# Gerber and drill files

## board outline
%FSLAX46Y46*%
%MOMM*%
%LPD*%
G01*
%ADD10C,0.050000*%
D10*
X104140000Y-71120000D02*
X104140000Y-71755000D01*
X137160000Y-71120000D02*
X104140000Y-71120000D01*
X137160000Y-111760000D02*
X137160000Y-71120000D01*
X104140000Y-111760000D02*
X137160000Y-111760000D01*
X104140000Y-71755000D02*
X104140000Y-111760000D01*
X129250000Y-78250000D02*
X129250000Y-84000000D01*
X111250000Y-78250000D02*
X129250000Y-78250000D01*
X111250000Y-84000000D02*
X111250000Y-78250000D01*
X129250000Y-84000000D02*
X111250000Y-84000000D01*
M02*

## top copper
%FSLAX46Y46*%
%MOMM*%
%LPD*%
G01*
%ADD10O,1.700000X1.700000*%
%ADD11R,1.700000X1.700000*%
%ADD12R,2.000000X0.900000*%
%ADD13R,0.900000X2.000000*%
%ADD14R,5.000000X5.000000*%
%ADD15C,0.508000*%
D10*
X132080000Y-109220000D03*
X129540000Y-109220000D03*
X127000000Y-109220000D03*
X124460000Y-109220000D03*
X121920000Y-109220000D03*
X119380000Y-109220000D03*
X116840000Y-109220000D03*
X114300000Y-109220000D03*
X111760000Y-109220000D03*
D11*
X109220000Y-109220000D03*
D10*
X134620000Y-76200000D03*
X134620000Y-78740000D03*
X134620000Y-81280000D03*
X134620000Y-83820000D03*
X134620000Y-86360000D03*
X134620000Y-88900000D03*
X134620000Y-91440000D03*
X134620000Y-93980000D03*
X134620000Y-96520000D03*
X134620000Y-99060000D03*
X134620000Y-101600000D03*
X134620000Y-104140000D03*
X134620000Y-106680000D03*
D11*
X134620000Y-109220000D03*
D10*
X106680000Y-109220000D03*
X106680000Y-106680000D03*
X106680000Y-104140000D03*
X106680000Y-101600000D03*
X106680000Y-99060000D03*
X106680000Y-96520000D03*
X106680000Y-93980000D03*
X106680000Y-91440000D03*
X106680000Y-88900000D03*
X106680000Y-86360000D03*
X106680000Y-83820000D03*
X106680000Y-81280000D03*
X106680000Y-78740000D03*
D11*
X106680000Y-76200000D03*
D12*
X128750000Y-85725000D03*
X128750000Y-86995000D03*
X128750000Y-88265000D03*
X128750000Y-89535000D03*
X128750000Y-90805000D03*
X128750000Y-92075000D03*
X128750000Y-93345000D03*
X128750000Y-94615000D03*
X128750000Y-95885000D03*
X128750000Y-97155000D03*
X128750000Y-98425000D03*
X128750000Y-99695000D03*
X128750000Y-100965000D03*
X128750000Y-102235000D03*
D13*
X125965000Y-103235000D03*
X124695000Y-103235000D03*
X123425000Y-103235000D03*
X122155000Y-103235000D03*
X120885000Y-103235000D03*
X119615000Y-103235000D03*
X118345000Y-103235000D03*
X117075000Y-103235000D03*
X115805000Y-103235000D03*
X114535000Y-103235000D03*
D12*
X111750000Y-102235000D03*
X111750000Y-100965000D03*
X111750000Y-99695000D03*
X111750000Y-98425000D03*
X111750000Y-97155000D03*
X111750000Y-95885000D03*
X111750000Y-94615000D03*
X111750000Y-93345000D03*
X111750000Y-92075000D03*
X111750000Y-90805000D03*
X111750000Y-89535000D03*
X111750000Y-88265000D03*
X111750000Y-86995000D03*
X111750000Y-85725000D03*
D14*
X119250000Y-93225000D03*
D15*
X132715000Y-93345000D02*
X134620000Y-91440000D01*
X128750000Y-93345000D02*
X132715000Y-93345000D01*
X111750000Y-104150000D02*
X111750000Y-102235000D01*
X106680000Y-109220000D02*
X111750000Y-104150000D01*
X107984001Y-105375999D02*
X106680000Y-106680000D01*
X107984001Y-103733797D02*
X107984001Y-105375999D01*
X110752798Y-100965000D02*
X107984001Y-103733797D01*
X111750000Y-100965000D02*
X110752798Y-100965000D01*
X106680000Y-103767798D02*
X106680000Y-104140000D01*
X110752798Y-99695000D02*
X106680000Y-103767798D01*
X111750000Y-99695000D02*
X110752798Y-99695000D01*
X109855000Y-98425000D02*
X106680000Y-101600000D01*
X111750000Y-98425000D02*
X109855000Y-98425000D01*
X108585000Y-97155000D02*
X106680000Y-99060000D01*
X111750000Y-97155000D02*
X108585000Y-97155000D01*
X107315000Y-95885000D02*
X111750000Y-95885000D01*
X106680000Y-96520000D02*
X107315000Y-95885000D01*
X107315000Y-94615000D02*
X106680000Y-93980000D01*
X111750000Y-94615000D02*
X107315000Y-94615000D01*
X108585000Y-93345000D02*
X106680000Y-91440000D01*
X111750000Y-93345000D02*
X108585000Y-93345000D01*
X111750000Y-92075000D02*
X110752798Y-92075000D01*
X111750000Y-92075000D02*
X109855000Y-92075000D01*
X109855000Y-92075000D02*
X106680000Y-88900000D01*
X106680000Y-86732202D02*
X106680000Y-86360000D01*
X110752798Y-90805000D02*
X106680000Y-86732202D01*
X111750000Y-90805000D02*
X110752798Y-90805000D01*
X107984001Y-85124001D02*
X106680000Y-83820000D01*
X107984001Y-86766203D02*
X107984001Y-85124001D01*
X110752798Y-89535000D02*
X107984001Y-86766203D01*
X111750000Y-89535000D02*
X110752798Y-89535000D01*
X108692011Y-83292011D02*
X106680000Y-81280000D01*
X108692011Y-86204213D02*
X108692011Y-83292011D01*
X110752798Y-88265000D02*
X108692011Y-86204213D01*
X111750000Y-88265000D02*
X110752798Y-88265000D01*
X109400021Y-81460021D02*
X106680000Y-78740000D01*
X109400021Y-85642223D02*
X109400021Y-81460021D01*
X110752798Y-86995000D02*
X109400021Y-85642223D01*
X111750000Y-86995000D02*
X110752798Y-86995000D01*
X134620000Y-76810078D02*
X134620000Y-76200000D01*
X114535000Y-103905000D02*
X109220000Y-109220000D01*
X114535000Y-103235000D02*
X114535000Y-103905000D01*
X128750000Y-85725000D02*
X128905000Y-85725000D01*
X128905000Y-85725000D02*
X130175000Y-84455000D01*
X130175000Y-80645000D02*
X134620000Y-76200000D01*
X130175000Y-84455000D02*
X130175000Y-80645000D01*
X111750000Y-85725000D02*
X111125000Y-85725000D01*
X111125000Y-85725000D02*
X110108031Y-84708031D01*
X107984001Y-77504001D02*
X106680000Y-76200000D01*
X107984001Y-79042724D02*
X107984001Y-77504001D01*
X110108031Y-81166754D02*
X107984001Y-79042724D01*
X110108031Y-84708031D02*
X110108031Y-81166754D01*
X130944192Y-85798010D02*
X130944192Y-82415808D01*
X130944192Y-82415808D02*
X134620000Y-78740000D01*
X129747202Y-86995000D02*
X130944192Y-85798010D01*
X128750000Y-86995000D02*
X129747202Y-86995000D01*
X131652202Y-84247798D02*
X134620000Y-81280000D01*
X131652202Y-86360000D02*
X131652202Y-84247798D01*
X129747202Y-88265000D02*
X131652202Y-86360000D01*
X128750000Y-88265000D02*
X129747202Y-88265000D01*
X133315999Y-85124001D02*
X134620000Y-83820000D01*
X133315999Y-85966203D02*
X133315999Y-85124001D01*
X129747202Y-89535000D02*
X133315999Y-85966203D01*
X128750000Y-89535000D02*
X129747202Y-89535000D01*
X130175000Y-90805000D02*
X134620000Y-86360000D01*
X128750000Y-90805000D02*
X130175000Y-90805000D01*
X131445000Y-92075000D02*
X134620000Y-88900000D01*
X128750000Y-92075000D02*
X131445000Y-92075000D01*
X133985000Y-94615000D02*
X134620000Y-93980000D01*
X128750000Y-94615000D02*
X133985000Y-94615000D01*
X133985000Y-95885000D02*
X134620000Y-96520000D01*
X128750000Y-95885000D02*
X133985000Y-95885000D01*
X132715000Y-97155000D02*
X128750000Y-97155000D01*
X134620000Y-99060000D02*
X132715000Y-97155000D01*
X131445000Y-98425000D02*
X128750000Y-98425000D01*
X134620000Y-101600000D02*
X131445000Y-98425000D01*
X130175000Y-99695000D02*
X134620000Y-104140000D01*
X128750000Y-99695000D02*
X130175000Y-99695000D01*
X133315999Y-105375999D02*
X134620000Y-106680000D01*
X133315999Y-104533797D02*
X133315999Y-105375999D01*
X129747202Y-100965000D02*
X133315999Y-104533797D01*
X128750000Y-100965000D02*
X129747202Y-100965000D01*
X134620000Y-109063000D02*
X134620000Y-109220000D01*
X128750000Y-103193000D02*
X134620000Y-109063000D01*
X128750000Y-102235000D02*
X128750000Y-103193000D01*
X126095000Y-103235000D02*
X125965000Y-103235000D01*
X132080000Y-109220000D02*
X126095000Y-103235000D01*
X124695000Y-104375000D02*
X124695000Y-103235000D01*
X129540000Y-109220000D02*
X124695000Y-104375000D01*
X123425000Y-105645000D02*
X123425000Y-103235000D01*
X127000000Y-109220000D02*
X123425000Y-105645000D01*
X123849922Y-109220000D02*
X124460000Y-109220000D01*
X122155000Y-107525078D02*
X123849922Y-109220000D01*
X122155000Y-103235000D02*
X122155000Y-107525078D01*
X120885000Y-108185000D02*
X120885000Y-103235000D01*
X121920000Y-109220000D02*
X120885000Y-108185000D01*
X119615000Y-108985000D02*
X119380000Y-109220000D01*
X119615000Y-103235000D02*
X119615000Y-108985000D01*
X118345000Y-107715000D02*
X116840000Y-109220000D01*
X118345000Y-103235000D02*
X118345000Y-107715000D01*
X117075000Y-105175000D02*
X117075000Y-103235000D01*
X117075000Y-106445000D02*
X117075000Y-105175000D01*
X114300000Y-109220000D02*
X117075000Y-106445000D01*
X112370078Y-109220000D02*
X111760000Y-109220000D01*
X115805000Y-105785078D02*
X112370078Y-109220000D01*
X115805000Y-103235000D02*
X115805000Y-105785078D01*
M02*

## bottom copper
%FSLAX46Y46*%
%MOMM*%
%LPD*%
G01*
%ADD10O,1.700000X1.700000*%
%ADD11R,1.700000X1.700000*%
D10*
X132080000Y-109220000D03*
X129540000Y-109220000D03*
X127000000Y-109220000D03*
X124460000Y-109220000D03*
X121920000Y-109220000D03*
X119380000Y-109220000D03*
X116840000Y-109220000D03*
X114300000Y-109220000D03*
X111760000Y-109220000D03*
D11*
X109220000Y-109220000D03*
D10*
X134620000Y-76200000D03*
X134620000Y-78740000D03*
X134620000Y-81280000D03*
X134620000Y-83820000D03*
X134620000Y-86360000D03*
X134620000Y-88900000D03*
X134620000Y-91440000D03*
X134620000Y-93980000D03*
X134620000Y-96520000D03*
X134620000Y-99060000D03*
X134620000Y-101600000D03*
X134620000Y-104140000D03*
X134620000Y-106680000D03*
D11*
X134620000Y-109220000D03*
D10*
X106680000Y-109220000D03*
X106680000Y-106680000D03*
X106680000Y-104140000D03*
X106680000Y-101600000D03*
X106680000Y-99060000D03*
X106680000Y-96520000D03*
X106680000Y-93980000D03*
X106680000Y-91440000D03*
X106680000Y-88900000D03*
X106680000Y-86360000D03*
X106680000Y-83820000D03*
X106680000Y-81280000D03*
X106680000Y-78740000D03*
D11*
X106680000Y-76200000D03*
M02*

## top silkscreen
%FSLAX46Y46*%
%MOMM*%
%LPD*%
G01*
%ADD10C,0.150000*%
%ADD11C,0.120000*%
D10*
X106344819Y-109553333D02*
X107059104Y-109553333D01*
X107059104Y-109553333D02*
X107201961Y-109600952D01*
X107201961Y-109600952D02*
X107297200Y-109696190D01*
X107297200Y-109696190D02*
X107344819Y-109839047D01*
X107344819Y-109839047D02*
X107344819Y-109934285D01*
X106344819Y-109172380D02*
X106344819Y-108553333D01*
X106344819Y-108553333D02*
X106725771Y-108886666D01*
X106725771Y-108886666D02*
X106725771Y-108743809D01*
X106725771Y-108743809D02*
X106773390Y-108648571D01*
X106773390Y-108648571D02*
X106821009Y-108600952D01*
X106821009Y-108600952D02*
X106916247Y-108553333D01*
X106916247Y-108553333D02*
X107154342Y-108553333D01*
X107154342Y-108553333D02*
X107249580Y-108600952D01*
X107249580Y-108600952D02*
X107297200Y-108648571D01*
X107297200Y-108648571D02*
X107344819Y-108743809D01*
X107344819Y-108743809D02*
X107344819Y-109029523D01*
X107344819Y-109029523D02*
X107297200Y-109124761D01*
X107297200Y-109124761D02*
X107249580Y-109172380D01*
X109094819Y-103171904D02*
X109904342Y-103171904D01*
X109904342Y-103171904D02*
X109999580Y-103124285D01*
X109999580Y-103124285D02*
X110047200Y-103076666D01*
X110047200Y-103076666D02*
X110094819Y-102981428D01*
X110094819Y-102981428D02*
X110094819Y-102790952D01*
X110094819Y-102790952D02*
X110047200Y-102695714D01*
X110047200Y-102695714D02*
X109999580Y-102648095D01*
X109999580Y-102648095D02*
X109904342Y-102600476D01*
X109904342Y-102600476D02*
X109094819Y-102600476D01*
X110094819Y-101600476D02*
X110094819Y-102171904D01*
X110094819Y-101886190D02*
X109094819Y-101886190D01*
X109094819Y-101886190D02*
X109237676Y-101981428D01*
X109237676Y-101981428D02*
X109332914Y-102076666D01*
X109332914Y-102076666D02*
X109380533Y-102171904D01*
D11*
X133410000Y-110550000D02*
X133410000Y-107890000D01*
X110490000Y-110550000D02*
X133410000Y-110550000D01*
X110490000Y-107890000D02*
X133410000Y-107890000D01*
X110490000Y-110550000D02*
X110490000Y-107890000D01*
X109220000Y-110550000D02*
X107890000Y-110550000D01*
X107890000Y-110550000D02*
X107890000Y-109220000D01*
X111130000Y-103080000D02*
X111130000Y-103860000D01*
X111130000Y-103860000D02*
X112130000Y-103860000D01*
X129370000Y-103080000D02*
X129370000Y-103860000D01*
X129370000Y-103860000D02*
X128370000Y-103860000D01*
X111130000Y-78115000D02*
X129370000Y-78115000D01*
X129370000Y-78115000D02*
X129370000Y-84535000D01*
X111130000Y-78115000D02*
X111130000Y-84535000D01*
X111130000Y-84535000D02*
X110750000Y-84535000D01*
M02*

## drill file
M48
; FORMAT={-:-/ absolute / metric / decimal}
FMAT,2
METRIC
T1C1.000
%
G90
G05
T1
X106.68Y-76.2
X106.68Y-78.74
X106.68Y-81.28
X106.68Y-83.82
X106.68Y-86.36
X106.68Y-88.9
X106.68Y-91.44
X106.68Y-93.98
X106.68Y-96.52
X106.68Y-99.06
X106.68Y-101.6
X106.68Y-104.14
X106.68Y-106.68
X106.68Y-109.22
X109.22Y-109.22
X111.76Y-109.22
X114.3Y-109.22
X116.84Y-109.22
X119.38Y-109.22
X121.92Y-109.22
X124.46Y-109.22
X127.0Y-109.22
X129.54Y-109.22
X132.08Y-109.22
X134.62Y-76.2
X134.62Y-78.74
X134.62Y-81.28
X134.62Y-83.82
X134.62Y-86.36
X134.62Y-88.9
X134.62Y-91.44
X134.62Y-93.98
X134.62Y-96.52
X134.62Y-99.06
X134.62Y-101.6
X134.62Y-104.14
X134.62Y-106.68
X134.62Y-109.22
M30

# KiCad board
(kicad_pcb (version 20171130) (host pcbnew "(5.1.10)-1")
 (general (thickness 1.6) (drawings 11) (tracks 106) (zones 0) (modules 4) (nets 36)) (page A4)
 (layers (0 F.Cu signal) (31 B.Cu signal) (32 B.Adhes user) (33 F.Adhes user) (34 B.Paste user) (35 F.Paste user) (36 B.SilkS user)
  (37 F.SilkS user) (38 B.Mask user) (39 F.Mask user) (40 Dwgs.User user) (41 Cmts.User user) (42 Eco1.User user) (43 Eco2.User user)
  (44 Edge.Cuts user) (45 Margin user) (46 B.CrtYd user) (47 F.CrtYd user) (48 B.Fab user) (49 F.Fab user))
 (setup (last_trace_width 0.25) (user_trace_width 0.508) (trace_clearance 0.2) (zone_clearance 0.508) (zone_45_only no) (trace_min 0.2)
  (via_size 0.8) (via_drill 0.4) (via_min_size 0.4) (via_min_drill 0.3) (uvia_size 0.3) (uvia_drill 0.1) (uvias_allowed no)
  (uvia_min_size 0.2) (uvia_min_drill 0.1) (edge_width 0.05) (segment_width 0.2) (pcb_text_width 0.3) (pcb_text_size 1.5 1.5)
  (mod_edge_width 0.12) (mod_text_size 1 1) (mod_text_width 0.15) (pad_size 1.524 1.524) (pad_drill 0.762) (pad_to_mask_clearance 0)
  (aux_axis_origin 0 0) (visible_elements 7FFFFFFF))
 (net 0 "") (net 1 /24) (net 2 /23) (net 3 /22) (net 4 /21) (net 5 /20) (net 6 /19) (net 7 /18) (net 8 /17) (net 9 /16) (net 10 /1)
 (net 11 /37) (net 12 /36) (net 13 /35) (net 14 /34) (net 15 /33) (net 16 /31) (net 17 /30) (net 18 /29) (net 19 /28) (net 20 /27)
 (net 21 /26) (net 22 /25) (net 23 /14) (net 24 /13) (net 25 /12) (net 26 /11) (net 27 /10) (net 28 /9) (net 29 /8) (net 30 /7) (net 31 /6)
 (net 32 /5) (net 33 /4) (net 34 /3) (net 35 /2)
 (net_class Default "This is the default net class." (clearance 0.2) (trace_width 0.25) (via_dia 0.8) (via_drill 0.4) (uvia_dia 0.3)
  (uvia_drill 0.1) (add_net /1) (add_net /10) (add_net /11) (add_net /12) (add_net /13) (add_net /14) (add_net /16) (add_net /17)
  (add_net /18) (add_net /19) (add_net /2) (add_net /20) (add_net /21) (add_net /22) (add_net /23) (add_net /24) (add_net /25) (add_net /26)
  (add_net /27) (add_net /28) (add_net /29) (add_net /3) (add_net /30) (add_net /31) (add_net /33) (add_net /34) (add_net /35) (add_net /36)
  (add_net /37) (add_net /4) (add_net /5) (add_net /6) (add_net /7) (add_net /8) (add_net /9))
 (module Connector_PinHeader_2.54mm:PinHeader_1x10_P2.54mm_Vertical (layer F.Cu) (at 109.22 109.22 90)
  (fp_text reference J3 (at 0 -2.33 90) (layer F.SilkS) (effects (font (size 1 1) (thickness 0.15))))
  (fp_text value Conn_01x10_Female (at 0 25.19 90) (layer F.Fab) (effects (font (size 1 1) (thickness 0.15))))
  (fp_line (start -1.33 24.19) (end 1.33 24.19) (layer F.SilkS) (width 0.12))
  (fp_line (start -1.33 1.27) (end -1.33 24.19) (layer F.SilkS) (width 0.12))
  (fp_line (start 1.33 1.27) (end 1.33 24.19) (layer F.SilkS) (width 0.12))
  (fp_line (start -1.33 1.27) (end 1.33 1.27) (layer F.SilkS) (width 0.12))
  (fp_line (start -1.33 0) (end -1.33 -1.33) (layer F.SilkS) (width 0.12))
  (fp_line (start -1.33 -1.33) (end 0 -1.33) (layer F.SilkS) (width 0.12))
  (pad 10 thru_hole oval (at 0 22.86 90) (size 1.7 1.7) (drill 1) (layers *.Cu *.Mask) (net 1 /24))
  (pad 9 thru_hole oval (at 0 20.32 90) (size 1.7 1.7) (drill 1) (layers *.Cu *.Mask) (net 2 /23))
  (pad 8 thru_hole oval (at 0 17.78 90) (size 1.7 1.7) (drill 1) (layers *.Cu *.Mask) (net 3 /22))
  (pad 7 thru_hole oval (at 0 15.24 90) (size 1.7 1.7) (drill 1) (layers *.Cu *.Mask) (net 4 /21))
  (pad 6 thru_hole oval (at 0 12.7 90) (size 1.7 1.7) (drill 1) (layers *.Cu *.Mask) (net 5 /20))
  (pad 5 thru_hole oval (at 0 10.16 90) (size 1.7 1.7) (drill 1) (layers *.Cu *.Mask) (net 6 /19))
  (pad 4 thru_hole oval (at 0 7.62 90) (size 1.7 1.7) (drill 1) (layers *.Cu *.Mask) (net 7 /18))
  (pad 3 thru_hole oval (at 0 5.08 90) (size 1.7 1.7) (drill 1) (layers *.Cu *.Mask) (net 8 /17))
  (pad 2 thru_hole oval (at 0 2.54 90) (size 1.7 1.7) (drill 1) (layers *.Cu *.Mask) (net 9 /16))
  (pad 1 thru_hole rect (at 0 0 90) (size 1.7 1.7) (drill 1) (layers *.Cu *.Mask) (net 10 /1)))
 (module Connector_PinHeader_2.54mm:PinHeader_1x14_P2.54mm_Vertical (layer B.Cu) (at 134.62 109.22)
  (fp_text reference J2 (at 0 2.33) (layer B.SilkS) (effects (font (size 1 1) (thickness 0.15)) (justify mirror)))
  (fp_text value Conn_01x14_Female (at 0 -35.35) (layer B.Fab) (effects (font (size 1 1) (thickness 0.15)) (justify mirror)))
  (pad 14 thru_hole oval (at 0 -33.02) (size 1.7 1.7) (drill 1) (layers *.Cu *.Mask) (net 10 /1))
  (pad 13 thru_hole oval (at 0 -30.48) (size 1.7 1.7) (drill 1) (layers *.Cu *.Mask) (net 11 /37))
  (pad 12 thru_hole oval (at 0 -27.94) (size 1.7 1.7) (drill 1) (layers *.Cu *.Mask) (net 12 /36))
  (pad 11 thru_hole oval (at 0 -25.4) (size 1.7 1.7) (drill 1) (layers *.Cu *.Mask) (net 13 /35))
  (pad 10 thru_hole oval (at 0 -22.86) (size 1.7 1.7) (drill 1) (layers *.Cu *.Mask) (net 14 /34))
  (pad 9 thru_hole oval (at 0 -20.32) (size 1.7 1.7) (drill 1) (layers *.Cu *.Mask) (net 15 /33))
  (pad 8 thru_hole oval (at 0 -17.78) (size 1.7 1.7) (drill 1) (layers *.Cu *.Mask))
  (pad 7 thru_hole oval (at 0 -15.24) (size 1.7 1.7) (drill 1) (layers *.Cu *.Mask) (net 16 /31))
  (pad 6 thru_hole oval (at 0 -12.7) (size 1.7 1.7) (drill 1) (layers *.Cu *.Mask) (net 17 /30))
  (pad 5 thru_hole oval (at 0 -10.16) (size 1.7 1.7) (drill 1) (layers *.Cu *.Mask) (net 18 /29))
  (pad 4 thru_hole oval (at 0 -7.62) (size 1.7 1.7) (drill 1) (layers *.Cu *.Mask) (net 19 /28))
  (pad 3 thru_hole oval (at 0 -5.08) (size 1.7 1.7) (drill 1) (layers *.Cu *.Mask) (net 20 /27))
  (pad 2 thru_hole oval (at 0 -2.54) (size 1.7 1.7) (drill 1) (layers *.Cu *.Mask) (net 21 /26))
  (pad 1 thru_hole rect (at 0 0) (size 1.7 1.7) (drill 1) (layers *.Cu *.Mask) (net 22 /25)))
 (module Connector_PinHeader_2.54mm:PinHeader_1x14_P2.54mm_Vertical (layer B.Cu) (at 106.68 76.2 180)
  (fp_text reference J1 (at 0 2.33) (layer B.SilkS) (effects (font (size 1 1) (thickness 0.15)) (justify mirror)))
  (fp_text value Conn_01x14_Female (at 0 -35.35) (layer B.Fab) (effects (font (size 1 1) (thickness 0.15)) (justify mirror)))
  (pad 14 thru_hole oval (at 0 -33.02 180) (size 1.7 1.7) (drill 1) (layers *.Cu *.Mask) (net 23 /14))
  (pad 13 thru_hole oval (at 0 -30.48 180) (size 1.7 1.7) (drill 1) (layers *.Cu *.Mask) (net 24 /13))
  (pad 12 thru_hole oval (at 0 -27.94 180) (size 1.7 1.7) (drill 1) (layers *.Cu *.Mask) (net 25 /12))
  (pad 11 thru_hole oval (at 0 -25.4 180) (size 1.7 1.7) (drill 1) (layers *.Cu *.Mask) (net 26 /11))
  (pad 10 thru_hole oval (at 0 -22.86 180) (size 1.7 1.7) (drill 1) (layers *.Cu *.Mask) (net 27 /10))
  (pad 9 thru_hole oval (at 0 -20.32 180) (size 1.7 1.7) (drill 1) (layers *.Cu *.Mask) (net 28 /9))
  (pad 8 thru_hole oval (at 0 -17.78 180) (size 1.7 1.7) (drill 1) (layers *.Cu *.Mask) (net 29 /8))
  (pad 7 thru_hole oval (at 0 -15.24 180) (size 1.7 1.7) (drill 1) (layers *.Cu *.Mask) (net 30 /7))
  (pad 6 thru_hole oval (at 0 -12.7 180) (size 1.7 1.7) (drill 1) (layers *.Cu *.Mask) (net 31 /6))
  (pad 5 thru_hole oval (at 0 -10.16 180) (size 1.7 1.7) (drill 1) (layers *.Cu *.Mask) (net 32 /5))
  (pad 4 thru_hole oval (at 0 -7.62 180) (size 1.7 1.7) (drill 1) (layers *.Cu *.Mask) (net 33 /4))
  (pad 3 thru_hole oval (at 0 -5.08 180) (size 1.7 1.7) (drill 1) (layers *.Cu *.Mask) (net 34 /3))
  (pad 2 thru_hole oval (at 0 -2.54 180) (size 1.7 1.7) (drill 1) (layers *.Cu *.Mask) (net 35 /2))
  (pad 1 thru_hole rect (at 0 0 180) (size 1.7 1.7) (drill 1) (layers *.Cu *.Mask) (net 10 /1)))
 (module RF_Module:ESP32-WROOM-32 (layer F.Cu) (at 120.25 93.98)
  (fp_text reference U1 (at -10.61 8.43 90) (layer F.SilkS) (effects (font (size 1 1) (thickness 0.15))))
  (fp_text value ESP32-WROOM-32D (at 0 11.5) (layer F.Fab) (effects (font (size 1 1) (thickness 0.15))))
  (fp_line (start -9.12 9.1) (end -9.12 9.88) (layer F.SilkS) (width 0.12))
  (fp_line (start -9.12 9.88) (end -8.12 9.88) (layer F.SilkS) (width 0.12))
  (fp_line (start 9.12 9.1) (end 9.12 9.88) (layer F.SilkS) (width 0.12))
  (fp_line (start 9.12 9.88) (end 8.12 9.88) (layer F.SilkS) (width 0.12))
  (fp_line (start -9.12 -15.865) (end 9.12 -15.865) (layer F.SilkS) (width 0.12))
  (fp_line (start 9.12 -15.865) (end 9.12 -9.445) (layer F.SilkS) (width 0.12))
  (fp_line (start -9.12 -15.865) (end -9.12 -9.445) (layer F.SilkS) (width 0.12))
  (fp_line (start -9.12 -9.445) (end -9.5 -9.445) (layer F.SilkS) (width 0.12))
  (pad 38 smd rect (at 8.5 -8.255) (size 2 0.9) (layers F.Cu F.Paste F.Mask) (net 10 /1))
  (pad 37 smd rect (at 8.5 -6.985) (size 2 0.9) (layers F.Cu F.Paste F.Mask) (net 11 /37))
  (pad 36 smd rect (at 8.5 -5.715) (size 2 0.9) (layers F.Cu F.Paste F.Mask) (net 12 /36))
  (pad 35 smd rect (at 8.5 -4.445) (size 2 0.9) (layers F.Cu F.Paste F.Mask) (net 13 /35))
  (pad 34 smd rect (at 8.5 -3.175) (size 2 0.9) (layers F.Cu F.Paste F.Mask) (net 14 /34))
  (pad 33 smd rect (at 8.5 -1.905) (size 2 0.9) (layers F.Cu F.Paste F.Mask) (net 15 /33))
  (pad 32 smd rect (at 8.5 -0.635) (size 2 0.9) (layers F.Cu F.Paste F.Mask))
  (pad 31 smd rect (at 8.5 0.635) (size 2 0.9) (layers F.Cu F.Paste F.Mask) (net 16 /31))
  (pad 30 smd rect (at 8.5 1.905) (size 2 0.9) (layers F.Cu F.Paste F.Mask) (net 17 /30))
  (pad 29 smd rect (at 8.5 3.175) (size 2 0.9) (layers F.Cu F.Paste F.Mask) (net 18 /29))
  (pad 28 smd rect (at 8.5 4.445) (size 2 0.9) (layers F.Cu F.Paste F.Mask) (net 19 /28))
  (pad 27 smd rect (at 8.5 5.715) (size 2 0.9) (layers F.Cu F.Paste F.Mask) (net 20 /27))
  (pad 26 smd rect (at 8.5 6.985) (size 2 0.9) (layers F.Cu F.Paste F.Mask) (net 21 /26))
  (pad 25 smd rect (at 8.5 8.255) (size 2 0.9) (layers F.Cu F.Paste F.Mask) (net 22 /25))
  (pad 24 smd rect (at 5.715 9.255 90) (size 2 0.9) (layers F.Cu F.Paste F.Mask) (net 1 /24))
  (pad 23 smd rect (at 4.445 9.255 90) (size 2 0.9) (layers F.Cu F.Paste F.Mask) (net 2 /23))
  (pad 22 smd rect (at 3.175 9.255 90) (size 2 0.9) (layers F.Cu F.Paste F.Mask) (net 3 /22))
  (pad 21 smd rect (at 1.905 9.255 90) (size 2 0.9) (layers F.Cu F.Paste F.Mask) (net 4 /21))
  (pad 20 smd rect (at 0.635 9.255 90) (size 2 0.9) (layers F.Cu F.Paste F.Mask) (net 5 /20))
  (pad 19 smd rect (at -0.635 9.255 90) (size 2 0.9) (layers F.Cu F.Paste F.Mask) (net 6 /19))
  (pad 18 smd rect (at -1.905 9.255 90) (size 2 0.9) (layers F.Cu F.Paste F.Mask) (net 7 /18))
  (pad 17 smd rect (at -3.175 9.255 90) (size 2 0.9) (layers F.Cu F.Paste F.Mask) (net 8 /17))
  (pad 16 smd rect (at -4.445 9.255 90) (size 2 0.9) (layers F.Cu F.Paste F.Mask) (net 9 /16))
  (pad 15 smd rect (at -5.715 9.255 90) (size 2 0.9) (layers F.Cu F.Paste F.Mask) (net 10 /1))
  (pad 14 smd rect (at -8.5 8.255) (size 2 0.9) (layers F.Cu F.Paste F.Mask) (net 23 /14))
  (pad 13 smd rect (at -8.5 6.985) (size 2 0.9) (layers F.Cu F.Paste F.Mask) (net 24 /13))
  (pad 12 smd rect (at -8.5 5.715) (size 2 0.9) (layers F.Cu F.Paste F.Mask) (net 25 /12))
  (pad 11 smd rect (at -8.5 4.445) (size 2 0.9) (layers F.Cu F.Paste F.Mask) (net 26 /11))
  (pad 10 smd rect (at -8.5 3.175) (size 2 0.9) (layers F.Cu F.Paste F.Mask) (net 27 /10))
  (pad 9 smd rect (at -8.5 1.905) (size 2 0.9) (layers F.Cu F.Paste F.Mask) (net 28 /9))
  (pad 8 smd rect (at -8.5 0.635) (size 2 0.9) (layers F.Cu F.Paste F.Mask) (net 29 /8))
  (pad 7 smd rect (at -8.5 -0.635) (size 2 0.9) (layers F.Cu F.Paste F.Mask) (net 30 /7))
  (pad 6 smd rect (at -8.5 -1.905) (size 2 0.9) (layers F.Cu F.Paste F.Mask) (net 31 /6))
  (pad 5 smd rect (at -8.5 -3.175) (size 2 0.9) (layers F.Cu F.Paste F.Mask) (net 32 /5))
  (pad 4 smd rect (at -8.5 -4.445) (size 2 0.9) (layers F.Cu F.Paste F.Mask) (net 33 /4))
  (pad 3 smd rect (at -8.5 -5.715) (size 2 0.9) (layers F.Cu F.Paste F.Mask) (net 34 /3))
  (pad 2 smd rect (at -8.5 -6.985) (size 2 0.9) (layers F.Cu F.Paste F.Mask) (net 35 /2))
  (pad 1 smd rect (at -8.5 -8.255) (size 2 0.9) (layers F.Cu F.Paste F.Mask) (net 10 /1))
  (pad 39 smd rect (at -1 -0.755) (size 5 5) (layers F.Cu F.Paste F.Mask) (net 10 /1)))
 (gr_line (start 104.14 71.12) (end 104.14 71.755) (layer Edge.Cuts) (width 0.05))
 (gr_line (start 137.16 71.12) (end 104.14 71.12) (layer Edge.Cuts) (width 0.05))
 (gr_line (start 137.16 111.76) (end 137.16 71.12) (layer Edge.Cuts) (width 0.05))
 (gr_line (start 104.14 111.76) (end 137.16 111.76) (layer Edge.Cuts) (width 0.05))
 (gr_line (start 104.14 71.755) (end 104.14 111.76) (layer Edge.Cuts) (width 0.05))
 (gr_line (start 129.25 78.25) (end 129.25 84) (layer Edge.Cuts) (width 0.05))
 (gr_line (start 111.25 78.25) (end 129.25 78.25) (layer Edge.Cuts) (width 0.05))
 (gr_line (start 111.25 84) (end 111.25 78.25) (layer Edge.Cuts) (width 0.05))
 (gr_line (start 129.25 84) (end 111.25 84) (layer Edge.Cuts) (width 0.05))
 (segment (start 132.715 93.345) (end 134.62 91.44) (width 0.508) (layer F.Cu) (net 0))
 (segment (start 128.75 93.345) (end 132.715 93.345) (width 0.508) (layer F.Cu) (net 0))
 (segment (start 111.75 104.15) (end 111.75 102.235) (width 0.508) (layer F.Cu) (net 23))
 (segment (start 106.68 109.22) (end 111.75 104.15) (width 0.508) (layer F.Cu) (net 23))
 (segment (start 107.984001 105.375999) (end 106.68 106.68) (width 0.508) (layer F.Cu) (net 24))
 (segment (start 107.984001 103.733797) (end 107.984001 105.375999) (width 0.508) (layer F.Cu) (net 24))
 (segment (start 110.752798 100.965) (end 107.984001 103.733797) (width 0.508) (layer F.Cu) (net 24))
 (segment (start 111.75 100.965) (end 110.752798 100.965) (width 0.508) (layer F.Cu) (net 24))
 (segment (start 106.68 103.767798) (end 106.68 104.14) (width 0.508) (layer F.Cu) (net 25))
 (segment (start 110.752798 99.695) (end 106.68 103.767798) (width 0.508) (layer F.Cu) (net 25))
 (segment (start 111.75 99.695) (end 110.752798 99.695) (width 0.508) (layer F.Cu) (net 25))
 (segment (start 109.855 98.425) (end 106.68 101.6) (width 0.508) (layer F.Cu) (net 26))
 (segment (start 111.75 98.425) (end 109.855 98.425) (width 0.508) (layer F.Cu) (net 26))
 (segment (start 108.585 97.155) (end 106.68 99.06) (width 0.508) (layer F.Cu) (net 27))
 (segment (start 111.75 97.155) (end 108.585 97.155) (width 0.508) (layer F.Cu) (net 27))
 (segment (start 107.315 95.885) (end 111.75 95.885) (width 0.508) (layer F.Cu) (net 28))
 (segment (start 106.68 96.52) (end 107.315 95.885) (width 0.508) (layer F.Cu) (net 28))
 (segment (start 107.315 94.615) (end 106.68 93.98) (width 0.508) (layer F.Cu) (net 29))
 (segment (start 111.75 94.615) (end 107.315 94.615) (width 0.508) (layer F.Cu) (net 29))
 (segment (start 108.585 93.345) (end 106.68 91.44) (width 0.508) (layer F.Cu) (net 30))
 (segment (start 111.75 93.345) (end 108.585 93.345) (width 0.508) (layer F.Cu) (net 30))
 (segment (start 111.75 92.075) (end 110.752798 92.075) (width 0.508) (layer F.Cu) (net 31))
 (segment (start 111.75 92.075) (end 109.855 92.075) (width 0.508) (layer F.Cu) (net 31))
 (segment (start 109.855 92.075) (end 106.68 88.9) (width 0.508) (layer F.Cu) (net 31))
 (segment (start 106.68 86.732202) (end 106.68 86.36) (width 0.508) (layer F.Cu) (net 32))
 (segment (start 110.752798 90.805) (end 106.68 86.732202) (width 0.508) (layer F.Cu) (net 32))
 (segment (start 111.75 90.805) (end 110.752798 90.805) (width 0.508) (layer F.Cu) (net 32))
 (segment (start 107.984001 85.124001) (end 106.68 83.82) (width 0.508) (layer F.Cu) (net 33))
 (segment (start 107.984001 86.766203) (end 107.984001 85.124001) (width 0.508) (layer F.Cu) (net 33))
 (segment (start 110.752798 89.535) (end 107.984001 86.766203) (width 0.508) (layer F.Cu) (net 33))
 (segment (start 111.75 89.535) (end 110.752798 89.535) (width 0.508) (layer F.Cu) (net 33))
 (segment (start 108.692011 83.292011) (end 106.68 81.28) (width 0.508) (layer F.Cu) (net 34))
 (segment (start 108.692011 86.204213) (end 108.692011 83.292011) (width 0.508) (layer F.Cu) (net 34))
 (segment (start 110.752798 88.265) (end 108.692011 86.204213) (width 0.508) (layer F.Cu) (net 34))
 (segment (start 111.75 88.265) (end 110.752798 88.265) (width 0.508) (layer F.Cu) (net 34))
 (segment (start 109.400021 81.460021) (end 106.68 78.74) (width 0.508) (layer F.Cu) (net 35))
 (segment (start 109.400021 85.642223) (end 109.400021 81.460021) (width 0.508) (layer F.Cu) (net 35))
 (segment (start 110.752798 86.995) (end 109.400021 85.642223) (width 0.508) (layer F.Cu) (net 35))
 (segment (start 111.75 86.995) (end 110.752798 86.995) (width 0.508) (layer F.Cu) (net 35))
 (segment (start 134.62 76.810078) (end 134.62 76.2) (width 0.508) (layer F.Cu) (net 10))
 (segment (start 114.535 103.905) (end 109.22 109.22) (width 0.508) (layer F.Cu) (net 10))
 (segment (start 114.535 103.235) (end 114.535 103.905) (width 0.508) (layer F.Cu) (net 10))
 (segment (start 128.75 85.725) (end 128.905 85.725) (width 0.508) (layer F.Cu) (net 10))
 (segment (start 128.905 85.725) (end 130.175 84.455) (width 0.508) (layer F.Cu) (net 10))
 (segment (start 130.175 80.645) (end 134.62 76.2) (width 0.508) (layer F.Cu) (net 10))
 (segment (start 130.175 84.455) (end 130.175 80.645) (width 0.508) (layer F.Cu) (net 10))
 (segment (start 111.75 85.725) (end 111.125 85.725) (width 0.508) (layer F.Cu) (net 10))
 (segment (start 111.125 85.725) (end 110.108031 84.708031) (width 0.508) (layer F.Cu) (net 10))
 (segment (start 107.984001 77.504001) (end 106.68 76.2) (width 0.508) (layer F.Cu) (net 10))
 (segment (start 107.984001 79.042724) (end 107.984001 77.504001) (width 0.508) (layer F.Cu) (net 10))
 (segment (start 110.108031 81.166754) (end 107.984001 79.042724) (width 0.508) (layer F.Cu) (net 10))
 (segment (start 110.108031 84.708031) (end 110.108031 81.166754) (width 0.508) (layer F.Cu) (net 10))
 (segment (start 130.944192 85.79801) (end 130.944192 82.415808) (width 0.508) (layer F.Cu) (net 11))
 (segment (start 130.944192 82.415808) (end 134.62 78.74) (width 0.508) (layer F.Cu) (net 11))
 (segment (start 129.747202 86.995) (end 130.944192 85.79801) (width 0.508) (layer F.Cu) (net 11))
 (segment (start 128.75 86.995) (end 129.747202 86.995) (width 0.508) (layer F.Cu) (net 11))
 (segment (start 131.652202 84.247798) (end 134.62 81.28) (width 0.508) (layer F.Cu) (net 12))
 (segment (start 131.652202 86.36) (end 131.652202 84.247798) (width 0.508) (layer F.Cu) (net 12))
 (segment (start 129.747202 88.265) (end 131.652202 86.36) (width 0.508) (layer F.Cu) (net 12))
 (segment (start 128.75 88.265) (end 129.747202 88.265) (width 0.508) (layer F.Cu) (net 12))
 (segment (start 133.315999 85.124001) (end 134.62 83.82) (width 0.508) (layer F.Cu) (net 13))
 (segment (start 133.315999 85.966203) (end 133.315999 85.124001) (width 0.508) (layer F.Cu) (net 13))
 (segment (start 129.747202 89.535) (end 133.315999 85.966203) (width 0.508) (layer F.Cu) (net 13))
 (segment (start 128.75 89.535) (end 129.747202 89.535) (width 0.508) (layer F.Cu) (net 13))
 (segment (start 130.175 90.805) (end 134.62 86.36) (width 0.508) (layer F.Cu) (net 14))
 (segment (start 128.75 90.805) (end 130.175 90.805) (width 0.508) (layer F.Cu) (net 14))
 (segment (start 131.445 92.075) (end 134.62 88.9) (width 0.508) (layer F.Cu) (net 15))
 (segment (start 128.75 92.075) (end 131.445 92.075) (width 0.508) (layer F.Cu) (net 15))
 (segment (start 133.985 94.615) (end 134.62 93.98) (width 0.508) (layer F.Cu) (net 16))
 (segment (start 128.75 94.615) (end 133.985 94.615) (width 0.508) (layer F.Cu) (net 16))
 (segment (start 133.985 95.885) (end 134.62 96.52) (width 0.508) (layer F.Cu) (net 17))
 (segment (start 128.75 95.885) (end 133.985 95.885) (width 0.508) (layer F.Cu) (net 17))
 (segment (start 132.715 97.155) (end 128.75 97.155) (width 0.508) (layer F.Cu) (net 18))
 (segment (start 134.62 99.06) (end 132.715 97.155) (width 0.508) (layer F.Cu) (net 18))
 (segment (start 131.445 98.425) (end 128.75 98.425) (width 0.508) (layer F.Cu) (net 19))
 (segment (start 134.62 101.6) (end 131.445 98.425) (width 0.508) (layer F.Cu) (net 19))
 (segment (start 130.175 99.695) (end 134.62 104.14) (width 0.508) (layer F.Cu) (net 20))
 (segment (start 128.75 99.695) (end 130.175 99.695) (width 0.508) (layer F.Cu) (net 20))
 (segment (start 133.315999 105.375999) (end 134.62 106.68) (width 0.508) (layer F.Cu) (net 21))
 (segment (start 133.315999 104.533797) (end 133.315999 105.375999) (width 0.508) (layer F.Cu) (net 21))
 (segment (start 129.747202 100.965) (end 133.315999 104.533797) (width 0.508) (layer F.Cu) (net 21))
 (segment (start 128.75 100.965) (end 129.747202 100.965) (width 0.508) (layer F.Cu) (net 21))
 (segment (start 134.62 109.063) (end 134.62 109.22) (width 0.508) (layer F.Cu) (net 22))
 (segment (start 128.75 103.193) (end 134.62 109.063) (width 0.508) (layer F.Cu) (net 22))
 (segment (start 128.75 102.235) (end 128.75 103.193) (width 0.508) (layer F.Cu) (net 22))
 (segment (start 126.095 103.235) (end 125.965 103.235) (width 0.508) (layer F.Cu) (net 1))
 (segment (start 132.08 109.22) (end 126.095 103.235) (width 0.508) (layer F.Cu) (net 1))
 (segment (start 124.695 104.375) (end 124.695 103.235) (width 0.508) (layer F.Cu) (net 2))
 (segment (start 129.54 109.22) (end 124.695 104.375) (width 0.508) (layer F.Cu) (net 2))
 (segment (start 123.425 105.645) (end 123.425 103.235) (width 0.508) (layer F.Cu) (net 3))
 (segment (start 127 109.22) (end 123.425 105.645) (width 0.508) (layer F.Cu) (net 3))
 (segment (start 123.849922 109.22) (end 124.46 109.22) (width 0.508) (layer F.Cu) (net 4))
 (segment (start 122.155 107.525078) (end 123.849922 109.22) (width 0.508) (layer F.Cu) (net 4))
 (segment (start 122.155 103.235) (end 122.155 107.525078) (width 0.508) (layer F.Cu) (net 4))
 (segment (start 120.885 108.185) (end 120.885 103.235) (width 0.508) (layer F.Cu) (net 5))
 (segment (start 121.92 109.22) (end 120.885 108.185) (width 0.508) (layer F.Cu) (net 5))
 (segment (start 119.615 108.985) (end 119.38 109.22) (width 0.508) (layer F.Cu) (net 6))
 (segment (start 119.615 103.235) (end 119.615 108.985) (width 0.508) (layer F.Cu) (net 6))
 (segment (start 118.345 107.715) (end 116.84 109.22) (width 0.508) (layer F.Cu) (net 7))
 (segment (start 118.345 103.235) (end 118.345 107.715) (width 0.508) (layer F.Cu) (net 7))
 (segment (start 117.075 105.175) (end 117.075 103.235) (width 0.508) (layer F.Cu) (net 8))
 (segment (start 117.075 106.445) (end 117.075 105.175) (width 0.508) (layer F.Cu) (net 8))
 (segment (start 114.3 109.22) (end 117.075 106.445) (width 0.508) (layer F.Cu) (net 8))
 (segment (start 112.370078 109.22) (end 111.76 109.22) (width 0.508) (layer F.Cu) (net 9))
 (segment (start 115.805 105.785078) (end 112.370078 109.22) (width 0.508) (layer F.Cu) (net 9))
 (segment (start 115.805 103.235) (end 115.805 105.785078) (width 0.508) (layer F.Cu) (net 9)))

